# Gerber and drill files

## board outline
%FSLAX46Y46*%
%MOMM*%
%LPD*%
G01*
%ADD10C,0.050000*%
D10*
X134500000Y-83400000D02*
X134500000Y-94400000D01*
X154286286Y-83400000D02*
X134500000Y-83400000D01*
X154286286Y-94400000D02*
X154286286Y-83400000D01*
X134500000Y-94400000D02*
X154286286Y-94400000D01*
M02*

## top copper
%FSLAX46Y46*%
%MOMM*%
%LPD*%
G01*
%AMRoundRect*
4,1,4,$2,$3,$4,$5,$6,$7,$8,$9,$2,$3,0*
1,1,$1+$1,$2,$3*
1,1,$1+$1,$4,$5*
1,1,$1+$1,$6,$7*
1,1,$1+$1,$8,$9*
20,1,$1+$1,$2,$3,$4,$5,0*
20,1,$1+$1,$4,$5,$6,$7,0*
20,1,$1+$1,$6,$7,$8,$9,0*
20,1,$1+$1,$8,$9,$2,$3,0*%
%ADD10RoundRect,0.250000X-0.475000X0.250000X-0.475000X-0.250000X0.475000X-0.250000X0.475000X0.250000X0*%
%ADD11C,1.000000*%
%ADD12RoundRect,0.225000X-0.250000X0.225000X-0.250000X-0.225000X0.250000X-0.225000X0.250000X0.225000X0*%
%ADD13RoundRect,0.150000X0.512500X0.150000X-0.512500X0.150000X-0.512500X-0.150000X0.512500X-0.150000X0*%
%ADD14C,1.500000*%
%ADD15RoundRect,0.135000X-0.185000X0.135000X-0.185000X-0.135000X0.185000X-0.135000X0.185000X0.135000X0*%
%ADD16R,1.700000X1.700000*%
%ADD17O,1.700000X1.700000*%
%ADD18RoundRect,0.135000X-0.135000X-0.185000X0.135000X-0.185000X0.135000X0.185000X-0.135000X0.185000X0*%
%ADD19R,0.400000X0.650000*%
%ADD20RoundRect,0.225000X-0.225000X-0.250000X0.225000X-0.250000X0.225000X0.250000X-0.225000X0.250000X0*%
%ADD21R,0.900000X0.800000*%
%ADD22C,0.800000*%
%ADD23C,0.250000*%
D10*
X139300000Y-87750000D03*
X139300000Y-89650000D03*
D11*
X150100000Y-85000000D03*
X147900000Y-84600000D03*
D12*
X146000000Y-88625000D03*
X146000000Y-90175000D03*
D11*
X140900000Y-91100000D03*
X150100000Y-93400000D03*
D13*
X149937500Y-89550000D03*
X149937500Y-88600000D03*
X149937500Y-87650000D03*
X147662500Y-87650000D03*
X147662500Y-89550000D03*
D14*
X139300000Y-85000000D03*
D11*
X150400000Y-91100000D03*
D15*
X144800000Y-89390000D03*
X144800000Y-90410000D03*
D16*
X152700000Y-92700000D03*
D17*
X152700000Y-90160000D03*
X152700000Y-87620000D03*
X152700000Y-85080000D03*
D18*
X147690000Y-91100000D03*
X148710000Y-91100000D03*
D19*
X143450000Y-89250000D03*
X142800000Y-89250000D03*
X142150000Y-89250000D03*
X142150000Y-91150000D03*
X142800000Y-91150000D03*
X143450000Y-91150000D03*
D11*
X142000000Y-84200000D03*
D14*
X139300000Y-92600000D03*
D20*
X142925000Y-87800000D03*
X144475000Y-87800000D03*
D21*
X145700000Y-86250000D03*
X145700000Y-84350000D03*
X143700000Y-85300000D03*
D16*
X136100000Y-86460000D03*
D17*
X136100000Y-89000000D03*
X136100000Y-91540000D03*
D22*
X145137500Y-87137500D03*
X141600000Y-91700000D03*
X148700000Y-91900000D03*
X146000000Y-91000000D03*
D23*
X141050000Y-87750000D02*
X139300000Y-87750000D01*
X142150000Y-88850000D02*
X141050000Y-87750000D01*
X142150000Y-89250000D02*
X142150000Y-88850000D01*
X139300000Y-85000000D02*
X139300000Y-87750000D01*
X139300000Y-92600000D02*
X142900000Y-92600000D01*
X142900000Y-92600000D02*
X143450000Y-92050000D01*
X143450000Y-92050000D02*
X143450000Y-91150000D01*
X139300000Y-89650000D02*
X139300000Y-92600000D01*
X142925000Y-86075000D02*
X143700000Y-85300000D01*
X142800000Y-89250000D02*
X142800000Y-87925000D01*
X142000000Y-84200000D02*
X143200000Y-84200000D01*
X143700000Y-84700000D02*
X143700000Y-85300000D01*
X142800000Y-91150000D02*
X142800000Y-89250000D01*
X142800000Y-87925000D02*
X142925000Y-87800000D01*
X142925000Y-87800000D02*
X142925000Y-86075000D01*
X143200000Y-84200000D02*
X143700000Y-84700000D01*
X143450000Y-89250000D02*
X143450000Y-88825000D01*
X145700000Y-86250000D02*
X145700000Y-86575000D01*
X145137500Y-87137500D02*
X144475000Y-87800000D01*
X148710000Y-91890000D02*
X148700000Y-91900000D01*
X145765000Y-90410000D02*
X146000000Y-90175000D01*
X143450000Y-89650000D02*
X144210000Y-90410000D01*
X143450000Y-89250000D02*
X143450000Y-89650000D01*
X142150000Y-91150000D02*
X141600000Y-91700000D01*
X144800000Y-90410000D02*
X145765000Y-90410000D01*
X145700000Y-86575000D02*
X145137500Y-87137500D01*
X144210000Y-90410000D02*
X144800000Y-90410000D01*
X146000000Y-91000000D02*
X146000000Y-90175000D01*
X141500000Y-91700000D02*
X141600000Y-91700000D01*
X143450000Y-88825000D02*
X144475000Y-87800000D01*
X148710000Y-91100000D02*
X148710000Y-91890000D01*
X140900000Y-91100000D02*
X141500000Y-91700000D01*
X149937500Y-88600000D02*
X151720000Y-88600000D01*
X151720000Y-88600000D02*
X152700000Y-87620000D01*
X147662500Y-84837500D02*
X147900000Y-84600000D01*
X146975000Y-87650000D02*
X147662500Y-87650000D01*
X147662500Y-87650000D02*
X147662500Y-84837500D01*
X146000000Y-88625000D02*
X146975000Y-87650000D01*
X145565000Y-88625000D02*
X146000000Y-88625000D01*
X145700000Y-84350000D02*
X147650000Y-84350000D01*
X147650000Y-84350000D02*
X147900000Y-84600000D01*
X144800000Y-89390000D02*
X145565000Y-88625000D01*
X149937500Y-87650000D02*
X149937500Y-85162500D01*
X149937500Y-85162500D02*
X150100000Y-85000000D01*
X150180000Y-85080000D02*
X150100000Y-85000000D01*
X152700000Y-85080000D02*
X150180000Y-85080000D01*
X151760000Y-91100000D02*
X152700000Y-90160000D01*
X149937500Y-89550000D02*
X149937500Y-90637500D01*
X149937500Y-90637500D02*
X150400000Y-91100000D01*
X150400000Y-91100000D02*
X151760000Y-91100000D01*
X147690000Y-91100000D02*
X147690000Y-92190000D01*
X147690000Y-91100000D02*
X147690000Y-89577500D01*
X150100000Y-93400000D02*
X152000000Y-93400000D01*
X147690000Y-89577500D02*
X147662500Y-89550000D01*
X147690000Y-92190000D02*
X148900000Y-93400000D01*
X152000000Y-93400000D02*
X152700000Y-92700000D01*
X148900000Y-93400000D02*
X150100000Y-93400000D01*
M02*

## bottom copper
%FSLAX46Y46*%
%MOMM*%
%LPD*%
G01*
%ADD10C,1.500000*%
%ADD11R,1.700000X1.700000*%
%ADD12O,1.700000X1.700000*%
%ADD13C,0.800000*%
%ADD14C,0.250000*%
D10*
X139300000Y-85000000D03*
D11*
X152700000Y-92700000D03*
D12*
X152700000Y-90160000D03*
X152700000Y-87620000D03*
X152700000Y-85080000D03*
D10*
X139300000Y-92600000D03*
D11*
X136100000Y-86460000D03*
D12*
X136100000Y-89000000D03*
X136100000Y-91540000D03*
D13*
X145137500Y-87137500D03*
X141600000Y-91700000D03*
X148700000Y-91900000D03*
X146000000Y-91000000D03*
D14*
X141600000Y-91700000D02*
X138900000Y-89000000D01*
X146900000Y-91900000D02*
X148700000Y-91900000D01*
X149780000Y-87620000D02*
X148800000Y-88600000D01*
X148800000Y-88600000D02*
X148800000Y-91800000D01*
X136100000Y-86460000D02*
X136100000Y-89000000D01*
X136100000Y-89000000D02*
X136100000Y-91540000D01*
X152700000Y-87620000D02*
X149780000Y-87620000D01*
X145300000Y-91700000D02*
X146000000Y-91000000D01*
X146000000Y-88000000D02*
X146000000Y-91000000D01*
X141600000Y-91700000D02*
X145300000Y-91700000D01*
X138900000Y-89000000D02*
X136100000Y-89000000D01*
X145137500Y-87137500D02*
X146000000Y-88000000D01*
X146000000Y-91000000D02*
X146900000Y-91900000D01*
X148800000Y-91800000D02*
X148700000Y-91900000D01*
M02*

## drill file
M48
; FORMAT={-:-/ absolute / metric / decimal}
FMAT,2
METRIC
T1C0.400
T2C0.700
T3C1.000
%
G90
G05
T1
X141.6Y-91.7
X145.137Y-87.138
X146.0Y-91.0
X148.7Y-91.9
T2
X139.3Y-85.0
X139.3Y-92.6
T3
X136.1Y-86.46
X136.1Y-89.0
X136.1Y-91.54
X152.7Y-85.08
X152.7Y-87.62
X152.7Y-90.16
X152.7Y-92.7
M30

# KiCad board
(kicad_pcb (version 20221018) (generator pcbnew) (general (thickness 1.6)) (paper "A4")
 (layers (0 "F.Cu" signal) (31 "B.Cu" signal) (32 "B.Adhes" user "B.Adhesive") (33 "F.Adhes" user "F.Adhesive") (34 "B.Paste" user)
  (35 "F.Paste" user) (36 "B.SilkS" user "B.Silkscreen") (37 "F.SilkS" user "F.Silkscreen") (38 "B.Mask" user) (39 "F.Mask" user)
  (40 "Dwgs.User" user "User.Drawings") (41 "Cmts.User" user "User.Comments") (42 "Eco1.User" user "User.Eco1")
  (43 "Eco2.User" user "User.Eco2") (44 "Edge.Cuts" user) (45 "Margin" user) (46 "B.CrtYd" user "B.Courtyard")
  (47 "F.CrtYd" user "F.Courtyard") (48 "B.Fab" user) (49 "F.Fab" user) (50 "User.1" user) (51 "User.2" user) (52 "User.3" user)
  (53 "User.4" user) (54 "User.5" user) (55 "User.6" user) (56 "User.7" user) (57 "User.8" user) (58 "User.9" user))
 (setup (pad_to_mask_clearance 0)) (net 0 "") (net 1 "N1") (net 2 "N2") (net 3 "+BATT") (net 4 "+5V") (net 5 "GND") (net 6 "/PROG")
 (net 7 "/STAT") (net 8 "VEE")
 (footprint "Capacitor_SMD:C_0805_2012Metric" (layer "F.Cu") (at 139.3 88.7 -90)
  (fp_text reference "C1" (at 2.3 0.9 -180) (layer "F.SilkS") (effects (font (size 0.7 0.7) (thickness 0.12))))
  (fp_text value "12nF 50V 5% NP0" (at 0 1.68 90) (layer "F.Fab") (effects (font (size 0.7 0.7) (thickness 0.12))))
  (pad "1" smd roundrect (at -0.95 0 270) (size 1 1.45) (layers "F.Cu" "F.Paste" "F.Mask") (roundrect_rratio 0.25) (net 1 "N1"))
  (pad "2" smd roundrect (at 0.95 0 270) (size 1 1.45) (layers "F.Cu" "F.Paste" "F.Mask") (roundrect_rratio 0.25) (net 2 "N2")))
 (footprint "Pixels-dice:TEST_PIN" (layer "F.Cu") (at 150.1 85)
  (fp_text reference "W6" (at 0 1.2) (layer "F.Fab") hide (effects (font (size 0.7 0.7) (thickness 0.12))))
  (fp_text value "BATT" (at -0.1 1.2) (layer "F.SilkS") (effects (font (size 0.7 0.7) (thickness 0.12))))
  (pad "1" smd circle (at 0 0) (size 1 1) (layers "F.Cu" "F.Mask") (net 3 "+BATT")))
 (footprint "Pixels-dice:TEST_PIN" (layer "F.Cu") (at 147.9 84.6)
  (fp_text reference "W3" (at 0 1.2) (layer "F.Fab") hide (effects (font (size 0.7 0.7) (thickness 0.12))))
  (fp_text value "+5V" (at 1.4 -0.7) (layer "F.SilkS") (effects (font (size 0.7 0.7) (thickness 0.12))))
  (pad "1" smd circle (at 0 0) (size 1 1) (layers "F.Cu" "F.Mask") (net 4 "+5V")))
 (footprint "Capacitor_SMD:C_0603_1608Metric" (layer "F.Cu") (at 146 89.4 -90)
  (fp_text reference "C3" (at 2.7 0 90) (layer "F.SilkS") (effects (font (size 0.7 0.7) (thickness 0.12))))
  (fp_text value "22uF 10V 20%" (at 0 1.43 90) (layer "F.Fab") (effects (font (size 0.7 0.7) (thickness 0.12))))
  (pad "1" smd roundrect (at -0.775 0 270) (size 0.9 0.95) (layers "F.Cu" "F.Paste" "F.Mask") (roundrect_rratio 0.25) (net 4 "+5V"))
  (pad "2" smd roundrect (at 0.775 0 270) (size 0.9 0.95) (layers "F.Cu" "F.Paste" "F.Mask") (roundrect_rratio 0.25) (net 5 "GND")))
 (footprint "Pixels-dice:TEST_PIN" (layer "F.Cu") (at 140.9 91.1)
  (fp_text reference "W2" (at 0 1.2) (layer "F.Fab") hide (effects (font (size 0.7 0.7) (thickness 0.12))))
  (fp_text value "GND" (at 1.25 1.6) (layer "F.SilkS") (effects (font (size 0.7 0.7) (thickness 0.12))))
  (pad "1" smd circle (at 0 0) (size 1 1) (layers "F.Cu" "F.Mask") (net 5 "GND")))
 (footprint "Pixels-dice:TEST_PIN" (layer "F.Cu") (at 150.1 93.4)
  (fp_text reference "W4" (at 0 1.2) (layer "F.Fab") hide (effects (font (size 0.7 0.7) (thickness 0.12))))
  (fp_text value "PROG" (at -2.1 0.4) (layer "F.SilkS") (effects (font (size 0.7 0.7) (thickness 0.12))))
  (pad "1" smd circle (at 0 0) (size 1 1) (layers "F.Cu" "F.Mask") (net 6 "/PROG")))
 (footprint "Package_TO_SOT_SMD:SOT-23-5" (layer "F.Cu") (at 148.8 88.6 180)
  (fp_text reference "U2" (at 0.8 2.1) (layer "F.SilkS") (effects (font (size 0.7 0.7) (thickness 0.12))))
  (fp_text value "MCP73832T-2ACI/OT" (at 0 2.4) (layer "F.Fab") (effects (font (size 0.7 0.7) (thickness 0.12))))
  (pad "1" smd roundrect (at -1.1375 -0.95 180) (size 1.325 0.6) (layers "F.Cu" "F.Paste" "F.Mask") (roundrect_rratio 0.25) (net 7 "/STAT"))
  (pad "2" smd roundrect (at -1.1375 0 180) (size 1.325 0.6) (layers "F.Cu" "F.Paste" "F.Mask") (roundrect_rratio 0.25) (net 5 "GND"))
  (pad "3" smd roundrect (at -1.1375 0.95 180) (size 1.325 0.6) (layers "F.Cu" "F.Paste" "F.Mask") (roundrect_rratio 0.25) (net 3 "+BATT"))
  (pad "4" smd roundrect (at 1.1375 0.95 180) (size 1.325 0.6) (layers "F.Cu" "F.Paste" "F.Mask") (roundrect_rratio 0.25) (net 4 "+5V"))
  (pad "5" smd roundrect (at 1.1375 -0.95 180) (size 1.325 0.6) (layers "F.Cu" "F.Paste" "F.Mask") (roundrect_rratio 0.25) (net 6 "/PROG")))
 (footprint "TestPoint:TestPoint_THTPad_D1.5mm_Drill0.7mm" (layer "F.Cu") (at 139.3 85)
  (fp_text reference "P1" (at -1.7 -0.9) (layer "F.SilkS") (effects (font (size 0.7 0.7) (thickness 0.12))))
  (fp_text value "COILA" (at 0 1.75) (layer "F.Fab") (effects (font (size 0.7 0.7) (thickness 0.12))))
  (pad "1" thru_hole circle (at 0 0) (size 1.5 1.5) (drill 0.7) (layers "*.Cu" "*.Mask") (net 1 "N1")))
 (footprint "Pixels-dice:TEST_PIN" (layer "F.Cu") (at 150.4 91.1)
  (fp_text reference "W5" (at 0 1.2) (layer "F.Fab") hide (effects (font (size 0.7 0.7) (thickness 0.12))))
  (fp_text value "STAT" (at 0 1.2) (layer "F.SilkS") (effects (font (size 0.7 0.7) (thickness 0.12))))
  (pad "1" smd circle (at 0 0) (size 1 1) (layers "F.Cu" "F.Mask") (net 7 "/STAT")))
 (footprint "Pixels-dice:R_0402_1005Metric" (layer "F.Cu") (at 144.8 89.9 -90)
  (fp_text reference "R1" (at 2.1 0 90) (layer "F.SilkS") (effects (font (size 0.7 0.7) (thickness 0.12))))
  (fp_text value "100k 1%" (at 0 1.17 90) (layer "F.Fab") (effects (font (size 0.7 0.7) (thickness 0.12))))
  (pad "1" smd roundrect (at -0.51 0 270) (size 0.54 0.64) (layers "F.Cu" "F.Paste" "F.Mask") (roundrect_rratio 0.25) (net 4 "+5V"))
  (pad "2" smd roundrect (at 0.51 0 270) (size 0.54 0.64) (layers "F.Cu" "F.Paste" "F.Mask") (roundrect_rratio 0.25) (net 5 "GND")))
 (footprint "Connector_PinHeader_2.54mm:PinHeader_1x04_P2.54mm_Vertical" (layer "F.Cu") (at 152.7 92.7 180)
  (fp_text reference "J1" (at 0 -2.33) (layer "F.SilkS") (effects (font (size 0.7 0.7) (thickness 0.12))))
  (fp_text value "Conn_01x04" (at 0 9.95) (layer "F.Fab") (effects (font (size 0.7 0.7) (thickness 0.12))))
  (pad "1" thru_hole rect (at 0 0 180) (size 1.7 1.7) (drill 1) (layers "*.Cu" "*.Mask") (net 6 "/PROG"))
  (pad "2" thru_hole oval (at 0 2.54 180) (size 1.7 1.7) (drill 1) (layers "*.Cu" "*.Mask") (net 7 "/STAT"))
  (pad "3" thru_hole oval (at 0 5.08 180) (size 1.7 1.7) (drill 1) (layers "*.Cu" "*.Mask") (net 5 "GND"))
  (pad "4" thru_hole oval (at 0 7.62 180) (size 1.7 1.7) (drill 1) (layers "*.Cu" "*.Mask") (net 3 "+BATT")))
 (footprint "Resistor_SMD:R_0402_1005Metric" (layer "F.Cu") (at 148.2 91.1)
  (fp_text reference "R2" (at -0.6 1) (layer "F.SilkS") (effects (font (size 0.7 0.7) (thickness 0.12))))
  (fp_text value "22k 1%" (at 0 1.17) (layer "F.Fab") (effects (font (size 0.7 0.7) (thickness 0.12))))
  (pad "1" smd roundrect (at -0.51 0) (size 0.54 0.64) (layers "F.Cu" "F.Paste" "F.Mask") (roundrect_rratio 0.25) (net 6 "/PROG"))
  (pad "2" smd roundrect (at 0.51 0) (size 0.54 0.64) (layers "F.Cu" "F.Paste" "F.Mask") (roundrect_rratio 0.25) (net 5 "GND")))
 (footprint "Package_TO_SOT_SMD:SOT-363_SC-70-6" (layer "F.Cu") (at 142.8 90.2 -90)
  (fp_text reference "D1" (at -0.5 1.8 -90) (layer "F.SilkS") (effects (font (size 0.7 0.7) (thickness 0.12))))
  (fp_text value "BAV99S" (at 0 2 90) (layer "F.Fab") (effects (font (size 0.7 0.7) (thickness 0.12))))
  (pad "1" smd rect (at -0.95 -0.65 270) (size 0.65 0.4) (layers "F.Cu" "F.Paste" "F.Mask") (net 5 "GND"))
  (pad "2" smd rect (at -0.95 0 270) (size 0.65 0.4) (layers "F.Cu" "F.Paste" "F.Mask") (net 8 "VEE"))
  (pad "3" smd rect (at -0.95 0.65 270) (size 0.65 0.4) (layers "F.Cu" "F.Paste" "F.Mask") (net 1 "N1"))
  (pad "4" smd rect (at 0.95 0.65 270) (size 0.65 0.4) (layers "F.Cu" "F.Paste" "F.Mask") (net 5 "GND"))
  (pad "5" smd rect (at 0.95 0 270) (size 0.65 0.4) (layers "F.Cu" "F.Paste" "F.Mask") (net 8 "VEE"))
  (pad "6" smd rect (at 0.95 -0.65 270) (size 0.65 0.4) (layers "F.Cu" "F.Paste" "F.Mask") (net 2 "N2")))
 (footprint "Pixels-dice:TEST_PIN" (layer "F.Cu") (at 142 84.2)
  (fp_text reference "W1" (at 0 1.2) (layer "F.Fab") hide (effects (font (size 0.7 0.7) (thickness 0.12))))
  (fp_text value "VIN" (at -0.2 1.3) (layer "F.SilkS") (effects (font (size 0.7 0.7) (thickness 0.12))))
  (pad "1" smd circle (at 0 0) (size 1 1) (layers "F.Cu" "F.Mask") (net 8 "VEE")))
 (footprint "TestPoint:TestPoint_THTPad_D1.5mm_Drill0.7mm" (layer "F.Cu") (at 139.3 92.6)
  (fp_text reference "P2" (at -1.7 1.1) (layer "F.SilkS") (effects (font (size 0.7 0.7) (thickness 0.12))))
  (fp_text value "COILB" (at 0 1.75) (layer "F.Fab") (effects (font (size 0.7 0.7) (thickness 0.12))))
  (pad "1" thru_hole circle (at 0 0) (size 1.5 1.5) (drill 0.7) (layers "*.Cu" "*.Mask") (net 2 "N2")))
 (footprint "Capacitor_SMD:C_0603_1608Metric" (layer "F.Cu") (at 143.7 87.8)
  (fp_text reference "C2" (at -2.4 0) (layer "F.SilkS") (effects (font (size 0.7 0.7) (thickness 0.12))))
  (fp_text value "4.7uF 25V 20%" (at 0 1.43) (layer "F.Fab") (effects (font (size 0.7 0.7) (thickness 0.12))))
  (pad "1" smd roundrect (at -0.775 0) (size 0.9 0.95) (layers "F.Cu" "F.Paste" "F.Mask") (roundrect_rratio 0.25) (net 8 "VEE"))
  (pad "2" smd roundrect (at 0.775 0) (size 0.9 0.95) (layers "F.Cu" "F.Paste" "F.Mask") (roundrect_rratio 0.25) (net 5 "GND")))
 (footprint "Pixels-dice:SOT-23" (layer "F.Cu") (at 144.7 85.3)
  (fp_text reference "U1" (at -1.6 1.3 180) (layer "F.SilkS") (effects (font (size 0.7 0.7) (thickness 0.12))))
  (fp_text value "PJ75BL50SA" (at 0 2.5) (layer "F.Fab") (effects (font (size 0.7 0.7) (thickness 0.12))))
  (pad "1" smd rect (at 1 0.95 180) (size 0.9 0.8) (layers "F.Cu" "F.Paste" "F.Mask") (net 5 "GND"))
  (pad "2" smd rect (at 1 -0.95 180) (size 0.9 0.8) (layers "F.Cu" "F.Paste" "F.Mask") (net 4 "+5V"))
  (pad "3" smd rect (at -1 0 180) (size 0.9 0.8) (layers "F.Cu" "F.Paste" "F.Mask") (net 8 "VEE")))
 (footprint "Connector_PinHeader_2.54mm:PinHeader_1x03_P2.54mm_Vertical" (layer "F.Cu") (at 136.1 86.46)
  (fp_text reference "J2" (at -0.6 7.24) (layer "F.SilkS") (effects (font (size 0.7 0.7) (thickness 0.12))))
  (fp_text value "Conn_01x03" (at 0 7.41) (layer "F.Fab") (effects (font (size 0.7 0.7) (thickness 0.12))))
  (pad "1" thru_hole rect (at 0 0) (size 1.7 1.7) (drill 1) (layers "*.Cu" "*.Mask") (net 5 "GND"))
  (pad "2" thru_hole oval (at 0 2.54) (size 1.7 1.7) (drill 1) (layers "*.Cu" "*.Mask") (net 5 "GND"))
  (pad "3" thru_hole oval (at 0 5.08) (size 1.7 1.7) (drill 1) (layers "*.Cu" "*.Mask") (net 5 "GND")))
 (gr_line (start 134.5 83.4) (end 134.5 94.4) (stroke (width 0.05) (type solid)) (layer "Edge.Cuts"))
 (gr_line (start 154.286286 83.4) (end 134.5 83.4) (stroke (width 0.05) (type solid)) (layer "Edge.Cuts"))
 (gr_line (start 154.286286 94.4) (end 154.286286 83.4) (stroke (width 0.05) (type solid)) (layer "Edge.Cuts"))
 (gr_line (start 134.5 94.4) (end 154.286286 94.4) (stroke (width 0.05) (type solid)) (layer "Edge.Cuts"))
 (segment (start 141.05 87.75) (end 139.3 87.75) (width 0.25) (layer "F.Cu") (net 1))
 (segment (start 142.15 88.85) (end 141.05 87.75) (width 0.25) (layer "F.Cu") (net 1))
 (segment (start 142.15 89.25) (end 142.15 88.85) (width 0.25) (layer "F.Cu") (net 1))
 (segment (start 139.3 85) (end 139.3 87.75) (width 0.25) (layer "F.Cu") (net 1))
 (segment (start 139.3 92.6) (end 142.9 92.6) (width 0.25) (layer "F.Cu") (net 2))
 (segment (start 142.9 92.6) (end 143.45 92.05) (width 0.25) (layer "F.Cu") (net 2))
 (segment (start 143.45 92.05) (end 143.45 91.15) (width 0.25) (layer "F.Cu") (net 2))
 (segment (start 139.3 89.65) (end 139.3 92.6) (width 0.25) (layer "F.Cu") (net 2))
 (segment (start 142.925 86.075) (end 143.7 85.3) (width 0.25) (layer "F.Cu") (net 8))
 (segment (start 142.8 89.25) (end 142.8 87.925) (width 0.25) (layer "F.Cu") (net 8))
 (segment (start 142 84.2) (end 143.2 84.2) (width 0.25) (layer "F.Cu") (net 8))
 (segment (start 143.7 84.7) (end 143.7 85.3) (width 0.25) (layer "F.Cu") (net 8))
 (segment (start 142.8 91.15) (end 142.8 89.25) (width 0.25) (layer "F.Cu") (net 8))
 (segment (start 142.8 87.925) (end 142.925 87.8) (width 0.25) (layer "F.Cu") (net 8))
 (segment (start 142.925 87.8) (end 142.925 86.075) (width 0.25) (layer "F.Cu") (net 8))
 (segment (start 143.2 84.2) (end 143.7 84.7) (width 0.25) (layer "F.Cu") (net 8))
 (segment (start 143.45 89.25) (end 143.45 88.825) (width 0.25) (layer "F.Cu") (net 5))
 (segment (start 145.7 86.25) (end 145.7 86.575) (width 0.25) (layer "F.Cu") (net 5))
 (segment (start 145.1375 87.1375) (end 144.475 87.8) (width 0.25) (layer "F.Cu") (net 5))
 (segment (start 148.71 91.89) (end 148.7 91.9) (width 0.25) (layer "F.Cu") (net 5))
 (segment (start 145.765 90.41) (end 146 90.175) (width 0.25) (layer "F.Cu") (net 5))
 (segment (start 143.45 89.65) (end 144.21 90.41) (width 0.25) (layer "F.Cu") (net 5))
 (segment (start 143.45 89.25) (end 143.45 89.65) (width 0.25) (layer "F.Cu") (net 5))
 (segment (start 142.15 91.15) (end 141.6 91.7) (width 0.25) (layer "F.Cu") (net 5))
 (segment (start 144.8 90.41) (end 145.765 90.41) (width 0.25) (layer "F.Cu") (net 5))
 (segment (start 145.7 86.575) (end 145.1375 87.1375) (width 0.25) (layer "F.Cu") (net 5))
 (segment (start 144.21 90.41) (end 144.8 90.41) (width 0.25) (layer "F.Cu") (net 5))
 (segment (start 146 91) (end 146 90.175) (width 0.25) (layer "F.Cu") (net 5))
 (segment (start 141.5 91.7) (end 141.6 91.7) (width 0.25) (layer "F.Cu") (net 5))
 (segment (start 143.45 88.825) (end 144.475 87.8) (width 0.25) (layer "F.Cu") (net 5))
 (segment (start 148.71 91.1) (end 148.71 91.89) (width 0.25) (layer "F.Cu") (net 5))
 (segment (start 140.9 91.1) (end 141.5 91.7) (width 0.25) (layer "F.Cu") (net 5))
 (segment (start 149.9375 88.6) (end 151.72 88.6) (width 0.25) (layer "F.Cu") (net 5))
 (segment (start 151.72 88.6) (end 152.7 87.62) (width 0.25) (layer "F.Cu") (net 5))
 (via (at 145.1375 87.1375) (size 0.8) (drill 0.4) (layers "F.Cu" "B.Cu") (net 5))
 (via (at 141.6 91.7) (size 0.8) (drill 0.4) (layers "F.Cu" "B.Cu") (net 5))
 (via (at 148.7 91.9) (size 0.8) (drill 0.4) (layers "F.Cu" "B.Cu") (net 5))
 (via (at 146 91) (size 0.8) (drill 0.4) (layers "F.Cu" "B.Cu") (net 5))
 (segment (start 141.6 91.7) (end 138.9 89) (width 0.25) (layer "B.Cu") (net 5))
 (segment (start 146.9 91.9) (end 148.7 91.9) (width 0.25) (layer "B.Cu") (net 5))
 (segment (start 149.78 87.62) (end 148.8 88.6) (width 0.25) (layer "B.Cu") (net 5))
 (segment (start 148.8 88.6) (end 148.8 91.8) (width 0.25) (layer "B.Cu") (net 5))
 (segment (start 136.1 86.46) (end 136.1 89) (width 0.25) (layer "B.Cu") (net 5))
 (segment (start 136.1 89) (end 136.1 91.54) (width 0.25) (layer "B.Cu") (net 5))
 (segment (start 152.7 87.62) (end 149.78 87.62) (width 0.25) (layer "B.Cu") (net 5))
 (segment (start 145.3 91.7) (end 146 91) (width 0.25) (layer "B.Cu") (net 5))
 (segment (start 146 88) (end 146 91) (width 0.25) (layer "B.Cu") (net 5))
 (segment (start 141.6 91.7) (end 145.3 91.7) (width 0.25) (layer "B.Cu") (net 5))
 (segment (start 138.9 89) (end 136.1 89) (width 0.25) (layer "B.Cu") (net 5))
 (segment (start 145.1375 87.1375) (end 146 88) (width 0.25) (layer "B.Cu") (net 5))
 (segment (start 146 91) (end 146.9 91.9) (width 0.25) (layer "B.Cu") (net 5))
 (segment (start 148.8 91.8) (end 148.7 91.9) (width 0.25) (layer "B.Cu") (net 5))
 (segment (start 147.6625 84.8375) (end 147.9 84.6) (width 0.25) (layer "F.Cu") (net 4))
 (segment (start 146.975 87.65) (end 147.6625 87.65) (width 0.25) (layer "F.Cu") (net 4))
 (segment (start 147.6625 87.65) (end 147.6625 84.8375) (width 0.25) (layer "F.Cu") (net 4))
 (segment (start 146 88.625) (end 146.975 87.65) (width 0.25) (layer "F.Cu") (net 4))
 (segment (start 145.565 88.625) (end 146 88.625) (width 0.25) (layer "F.Cu") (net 4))
 (segment (start 145.7 84.35) (end 147.65 84.35) (width 0.25) (layer "F.Cu") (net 4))
 (segment (start 147.65 84.35) (end 147.9 84.6) (width 0.25) (layer "F.Cu") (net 4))
 (segment (start 144.8 89.39) (end 145.565 88.625) (width 0.25) (layer "F.Cu") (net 4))
 (segment (start 149.9375 87.65) (end 149.9375 85.1625) (width 0.25) (layer "F.Cu") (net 3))
 (segment (start 149.9375 85.1625) (end 150.1 85) (width 0.25) (layer "F.Cu") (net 3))
 (segment (start 150.18 85.08) (end 150.1 85) (width 0.25) (layer "F.Cu") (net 3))
 (segment (start 152.7 85.08) (end 150.18 85.08) (width 0.25) (layer "F.Cu") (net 3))
 (segment (start 151.76 91.1) (end 152.7 90.16) (width 0.25) (layer "F.Cu") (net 7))
 (segment (start 149.9375 89.55) (end 149.9375 90.6375) (width 0.25) (layer "F.Cu") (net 7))
 (segment (start 149.9375 90.6375) (end 150.4 91.1) (width 0.25) (layer "F.Cu") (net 7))
 (segment (start 150.4 91.1) (end 151.76 91.1) (width 0.25) (layer "F.Cu") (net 7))
 (segment (start 147.69 91.1) (end 147.69 92.19) (width 0.25) (layer "F.Cu") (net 6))
 (segment (start 147.69 91.1) (end 147.69 89.5775) (width 0.25) (layer "F.Cu") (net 6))
 (segment (start 150.1 93.4) (end 152 93.4) (width 0.25) (layer "F.Cu") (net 6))
 (segment (start 147.69 89.5775) (end 147.6625 89.55) (width 0.25) (layer "F.Cu") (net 6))
 (segment (start 147.69 92.19) (end 148.9 93.4) (width 0.25) (layer "F.Cu") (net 6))
 (segment (start 152 93.4) (end 152.7 92.7) (width 0.25) (layer "F.Cu") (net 6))
 (segment (start 148.9 93.4) (end 150.1 93.4) (width 0.25) (layer "F.Cu") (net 6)))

